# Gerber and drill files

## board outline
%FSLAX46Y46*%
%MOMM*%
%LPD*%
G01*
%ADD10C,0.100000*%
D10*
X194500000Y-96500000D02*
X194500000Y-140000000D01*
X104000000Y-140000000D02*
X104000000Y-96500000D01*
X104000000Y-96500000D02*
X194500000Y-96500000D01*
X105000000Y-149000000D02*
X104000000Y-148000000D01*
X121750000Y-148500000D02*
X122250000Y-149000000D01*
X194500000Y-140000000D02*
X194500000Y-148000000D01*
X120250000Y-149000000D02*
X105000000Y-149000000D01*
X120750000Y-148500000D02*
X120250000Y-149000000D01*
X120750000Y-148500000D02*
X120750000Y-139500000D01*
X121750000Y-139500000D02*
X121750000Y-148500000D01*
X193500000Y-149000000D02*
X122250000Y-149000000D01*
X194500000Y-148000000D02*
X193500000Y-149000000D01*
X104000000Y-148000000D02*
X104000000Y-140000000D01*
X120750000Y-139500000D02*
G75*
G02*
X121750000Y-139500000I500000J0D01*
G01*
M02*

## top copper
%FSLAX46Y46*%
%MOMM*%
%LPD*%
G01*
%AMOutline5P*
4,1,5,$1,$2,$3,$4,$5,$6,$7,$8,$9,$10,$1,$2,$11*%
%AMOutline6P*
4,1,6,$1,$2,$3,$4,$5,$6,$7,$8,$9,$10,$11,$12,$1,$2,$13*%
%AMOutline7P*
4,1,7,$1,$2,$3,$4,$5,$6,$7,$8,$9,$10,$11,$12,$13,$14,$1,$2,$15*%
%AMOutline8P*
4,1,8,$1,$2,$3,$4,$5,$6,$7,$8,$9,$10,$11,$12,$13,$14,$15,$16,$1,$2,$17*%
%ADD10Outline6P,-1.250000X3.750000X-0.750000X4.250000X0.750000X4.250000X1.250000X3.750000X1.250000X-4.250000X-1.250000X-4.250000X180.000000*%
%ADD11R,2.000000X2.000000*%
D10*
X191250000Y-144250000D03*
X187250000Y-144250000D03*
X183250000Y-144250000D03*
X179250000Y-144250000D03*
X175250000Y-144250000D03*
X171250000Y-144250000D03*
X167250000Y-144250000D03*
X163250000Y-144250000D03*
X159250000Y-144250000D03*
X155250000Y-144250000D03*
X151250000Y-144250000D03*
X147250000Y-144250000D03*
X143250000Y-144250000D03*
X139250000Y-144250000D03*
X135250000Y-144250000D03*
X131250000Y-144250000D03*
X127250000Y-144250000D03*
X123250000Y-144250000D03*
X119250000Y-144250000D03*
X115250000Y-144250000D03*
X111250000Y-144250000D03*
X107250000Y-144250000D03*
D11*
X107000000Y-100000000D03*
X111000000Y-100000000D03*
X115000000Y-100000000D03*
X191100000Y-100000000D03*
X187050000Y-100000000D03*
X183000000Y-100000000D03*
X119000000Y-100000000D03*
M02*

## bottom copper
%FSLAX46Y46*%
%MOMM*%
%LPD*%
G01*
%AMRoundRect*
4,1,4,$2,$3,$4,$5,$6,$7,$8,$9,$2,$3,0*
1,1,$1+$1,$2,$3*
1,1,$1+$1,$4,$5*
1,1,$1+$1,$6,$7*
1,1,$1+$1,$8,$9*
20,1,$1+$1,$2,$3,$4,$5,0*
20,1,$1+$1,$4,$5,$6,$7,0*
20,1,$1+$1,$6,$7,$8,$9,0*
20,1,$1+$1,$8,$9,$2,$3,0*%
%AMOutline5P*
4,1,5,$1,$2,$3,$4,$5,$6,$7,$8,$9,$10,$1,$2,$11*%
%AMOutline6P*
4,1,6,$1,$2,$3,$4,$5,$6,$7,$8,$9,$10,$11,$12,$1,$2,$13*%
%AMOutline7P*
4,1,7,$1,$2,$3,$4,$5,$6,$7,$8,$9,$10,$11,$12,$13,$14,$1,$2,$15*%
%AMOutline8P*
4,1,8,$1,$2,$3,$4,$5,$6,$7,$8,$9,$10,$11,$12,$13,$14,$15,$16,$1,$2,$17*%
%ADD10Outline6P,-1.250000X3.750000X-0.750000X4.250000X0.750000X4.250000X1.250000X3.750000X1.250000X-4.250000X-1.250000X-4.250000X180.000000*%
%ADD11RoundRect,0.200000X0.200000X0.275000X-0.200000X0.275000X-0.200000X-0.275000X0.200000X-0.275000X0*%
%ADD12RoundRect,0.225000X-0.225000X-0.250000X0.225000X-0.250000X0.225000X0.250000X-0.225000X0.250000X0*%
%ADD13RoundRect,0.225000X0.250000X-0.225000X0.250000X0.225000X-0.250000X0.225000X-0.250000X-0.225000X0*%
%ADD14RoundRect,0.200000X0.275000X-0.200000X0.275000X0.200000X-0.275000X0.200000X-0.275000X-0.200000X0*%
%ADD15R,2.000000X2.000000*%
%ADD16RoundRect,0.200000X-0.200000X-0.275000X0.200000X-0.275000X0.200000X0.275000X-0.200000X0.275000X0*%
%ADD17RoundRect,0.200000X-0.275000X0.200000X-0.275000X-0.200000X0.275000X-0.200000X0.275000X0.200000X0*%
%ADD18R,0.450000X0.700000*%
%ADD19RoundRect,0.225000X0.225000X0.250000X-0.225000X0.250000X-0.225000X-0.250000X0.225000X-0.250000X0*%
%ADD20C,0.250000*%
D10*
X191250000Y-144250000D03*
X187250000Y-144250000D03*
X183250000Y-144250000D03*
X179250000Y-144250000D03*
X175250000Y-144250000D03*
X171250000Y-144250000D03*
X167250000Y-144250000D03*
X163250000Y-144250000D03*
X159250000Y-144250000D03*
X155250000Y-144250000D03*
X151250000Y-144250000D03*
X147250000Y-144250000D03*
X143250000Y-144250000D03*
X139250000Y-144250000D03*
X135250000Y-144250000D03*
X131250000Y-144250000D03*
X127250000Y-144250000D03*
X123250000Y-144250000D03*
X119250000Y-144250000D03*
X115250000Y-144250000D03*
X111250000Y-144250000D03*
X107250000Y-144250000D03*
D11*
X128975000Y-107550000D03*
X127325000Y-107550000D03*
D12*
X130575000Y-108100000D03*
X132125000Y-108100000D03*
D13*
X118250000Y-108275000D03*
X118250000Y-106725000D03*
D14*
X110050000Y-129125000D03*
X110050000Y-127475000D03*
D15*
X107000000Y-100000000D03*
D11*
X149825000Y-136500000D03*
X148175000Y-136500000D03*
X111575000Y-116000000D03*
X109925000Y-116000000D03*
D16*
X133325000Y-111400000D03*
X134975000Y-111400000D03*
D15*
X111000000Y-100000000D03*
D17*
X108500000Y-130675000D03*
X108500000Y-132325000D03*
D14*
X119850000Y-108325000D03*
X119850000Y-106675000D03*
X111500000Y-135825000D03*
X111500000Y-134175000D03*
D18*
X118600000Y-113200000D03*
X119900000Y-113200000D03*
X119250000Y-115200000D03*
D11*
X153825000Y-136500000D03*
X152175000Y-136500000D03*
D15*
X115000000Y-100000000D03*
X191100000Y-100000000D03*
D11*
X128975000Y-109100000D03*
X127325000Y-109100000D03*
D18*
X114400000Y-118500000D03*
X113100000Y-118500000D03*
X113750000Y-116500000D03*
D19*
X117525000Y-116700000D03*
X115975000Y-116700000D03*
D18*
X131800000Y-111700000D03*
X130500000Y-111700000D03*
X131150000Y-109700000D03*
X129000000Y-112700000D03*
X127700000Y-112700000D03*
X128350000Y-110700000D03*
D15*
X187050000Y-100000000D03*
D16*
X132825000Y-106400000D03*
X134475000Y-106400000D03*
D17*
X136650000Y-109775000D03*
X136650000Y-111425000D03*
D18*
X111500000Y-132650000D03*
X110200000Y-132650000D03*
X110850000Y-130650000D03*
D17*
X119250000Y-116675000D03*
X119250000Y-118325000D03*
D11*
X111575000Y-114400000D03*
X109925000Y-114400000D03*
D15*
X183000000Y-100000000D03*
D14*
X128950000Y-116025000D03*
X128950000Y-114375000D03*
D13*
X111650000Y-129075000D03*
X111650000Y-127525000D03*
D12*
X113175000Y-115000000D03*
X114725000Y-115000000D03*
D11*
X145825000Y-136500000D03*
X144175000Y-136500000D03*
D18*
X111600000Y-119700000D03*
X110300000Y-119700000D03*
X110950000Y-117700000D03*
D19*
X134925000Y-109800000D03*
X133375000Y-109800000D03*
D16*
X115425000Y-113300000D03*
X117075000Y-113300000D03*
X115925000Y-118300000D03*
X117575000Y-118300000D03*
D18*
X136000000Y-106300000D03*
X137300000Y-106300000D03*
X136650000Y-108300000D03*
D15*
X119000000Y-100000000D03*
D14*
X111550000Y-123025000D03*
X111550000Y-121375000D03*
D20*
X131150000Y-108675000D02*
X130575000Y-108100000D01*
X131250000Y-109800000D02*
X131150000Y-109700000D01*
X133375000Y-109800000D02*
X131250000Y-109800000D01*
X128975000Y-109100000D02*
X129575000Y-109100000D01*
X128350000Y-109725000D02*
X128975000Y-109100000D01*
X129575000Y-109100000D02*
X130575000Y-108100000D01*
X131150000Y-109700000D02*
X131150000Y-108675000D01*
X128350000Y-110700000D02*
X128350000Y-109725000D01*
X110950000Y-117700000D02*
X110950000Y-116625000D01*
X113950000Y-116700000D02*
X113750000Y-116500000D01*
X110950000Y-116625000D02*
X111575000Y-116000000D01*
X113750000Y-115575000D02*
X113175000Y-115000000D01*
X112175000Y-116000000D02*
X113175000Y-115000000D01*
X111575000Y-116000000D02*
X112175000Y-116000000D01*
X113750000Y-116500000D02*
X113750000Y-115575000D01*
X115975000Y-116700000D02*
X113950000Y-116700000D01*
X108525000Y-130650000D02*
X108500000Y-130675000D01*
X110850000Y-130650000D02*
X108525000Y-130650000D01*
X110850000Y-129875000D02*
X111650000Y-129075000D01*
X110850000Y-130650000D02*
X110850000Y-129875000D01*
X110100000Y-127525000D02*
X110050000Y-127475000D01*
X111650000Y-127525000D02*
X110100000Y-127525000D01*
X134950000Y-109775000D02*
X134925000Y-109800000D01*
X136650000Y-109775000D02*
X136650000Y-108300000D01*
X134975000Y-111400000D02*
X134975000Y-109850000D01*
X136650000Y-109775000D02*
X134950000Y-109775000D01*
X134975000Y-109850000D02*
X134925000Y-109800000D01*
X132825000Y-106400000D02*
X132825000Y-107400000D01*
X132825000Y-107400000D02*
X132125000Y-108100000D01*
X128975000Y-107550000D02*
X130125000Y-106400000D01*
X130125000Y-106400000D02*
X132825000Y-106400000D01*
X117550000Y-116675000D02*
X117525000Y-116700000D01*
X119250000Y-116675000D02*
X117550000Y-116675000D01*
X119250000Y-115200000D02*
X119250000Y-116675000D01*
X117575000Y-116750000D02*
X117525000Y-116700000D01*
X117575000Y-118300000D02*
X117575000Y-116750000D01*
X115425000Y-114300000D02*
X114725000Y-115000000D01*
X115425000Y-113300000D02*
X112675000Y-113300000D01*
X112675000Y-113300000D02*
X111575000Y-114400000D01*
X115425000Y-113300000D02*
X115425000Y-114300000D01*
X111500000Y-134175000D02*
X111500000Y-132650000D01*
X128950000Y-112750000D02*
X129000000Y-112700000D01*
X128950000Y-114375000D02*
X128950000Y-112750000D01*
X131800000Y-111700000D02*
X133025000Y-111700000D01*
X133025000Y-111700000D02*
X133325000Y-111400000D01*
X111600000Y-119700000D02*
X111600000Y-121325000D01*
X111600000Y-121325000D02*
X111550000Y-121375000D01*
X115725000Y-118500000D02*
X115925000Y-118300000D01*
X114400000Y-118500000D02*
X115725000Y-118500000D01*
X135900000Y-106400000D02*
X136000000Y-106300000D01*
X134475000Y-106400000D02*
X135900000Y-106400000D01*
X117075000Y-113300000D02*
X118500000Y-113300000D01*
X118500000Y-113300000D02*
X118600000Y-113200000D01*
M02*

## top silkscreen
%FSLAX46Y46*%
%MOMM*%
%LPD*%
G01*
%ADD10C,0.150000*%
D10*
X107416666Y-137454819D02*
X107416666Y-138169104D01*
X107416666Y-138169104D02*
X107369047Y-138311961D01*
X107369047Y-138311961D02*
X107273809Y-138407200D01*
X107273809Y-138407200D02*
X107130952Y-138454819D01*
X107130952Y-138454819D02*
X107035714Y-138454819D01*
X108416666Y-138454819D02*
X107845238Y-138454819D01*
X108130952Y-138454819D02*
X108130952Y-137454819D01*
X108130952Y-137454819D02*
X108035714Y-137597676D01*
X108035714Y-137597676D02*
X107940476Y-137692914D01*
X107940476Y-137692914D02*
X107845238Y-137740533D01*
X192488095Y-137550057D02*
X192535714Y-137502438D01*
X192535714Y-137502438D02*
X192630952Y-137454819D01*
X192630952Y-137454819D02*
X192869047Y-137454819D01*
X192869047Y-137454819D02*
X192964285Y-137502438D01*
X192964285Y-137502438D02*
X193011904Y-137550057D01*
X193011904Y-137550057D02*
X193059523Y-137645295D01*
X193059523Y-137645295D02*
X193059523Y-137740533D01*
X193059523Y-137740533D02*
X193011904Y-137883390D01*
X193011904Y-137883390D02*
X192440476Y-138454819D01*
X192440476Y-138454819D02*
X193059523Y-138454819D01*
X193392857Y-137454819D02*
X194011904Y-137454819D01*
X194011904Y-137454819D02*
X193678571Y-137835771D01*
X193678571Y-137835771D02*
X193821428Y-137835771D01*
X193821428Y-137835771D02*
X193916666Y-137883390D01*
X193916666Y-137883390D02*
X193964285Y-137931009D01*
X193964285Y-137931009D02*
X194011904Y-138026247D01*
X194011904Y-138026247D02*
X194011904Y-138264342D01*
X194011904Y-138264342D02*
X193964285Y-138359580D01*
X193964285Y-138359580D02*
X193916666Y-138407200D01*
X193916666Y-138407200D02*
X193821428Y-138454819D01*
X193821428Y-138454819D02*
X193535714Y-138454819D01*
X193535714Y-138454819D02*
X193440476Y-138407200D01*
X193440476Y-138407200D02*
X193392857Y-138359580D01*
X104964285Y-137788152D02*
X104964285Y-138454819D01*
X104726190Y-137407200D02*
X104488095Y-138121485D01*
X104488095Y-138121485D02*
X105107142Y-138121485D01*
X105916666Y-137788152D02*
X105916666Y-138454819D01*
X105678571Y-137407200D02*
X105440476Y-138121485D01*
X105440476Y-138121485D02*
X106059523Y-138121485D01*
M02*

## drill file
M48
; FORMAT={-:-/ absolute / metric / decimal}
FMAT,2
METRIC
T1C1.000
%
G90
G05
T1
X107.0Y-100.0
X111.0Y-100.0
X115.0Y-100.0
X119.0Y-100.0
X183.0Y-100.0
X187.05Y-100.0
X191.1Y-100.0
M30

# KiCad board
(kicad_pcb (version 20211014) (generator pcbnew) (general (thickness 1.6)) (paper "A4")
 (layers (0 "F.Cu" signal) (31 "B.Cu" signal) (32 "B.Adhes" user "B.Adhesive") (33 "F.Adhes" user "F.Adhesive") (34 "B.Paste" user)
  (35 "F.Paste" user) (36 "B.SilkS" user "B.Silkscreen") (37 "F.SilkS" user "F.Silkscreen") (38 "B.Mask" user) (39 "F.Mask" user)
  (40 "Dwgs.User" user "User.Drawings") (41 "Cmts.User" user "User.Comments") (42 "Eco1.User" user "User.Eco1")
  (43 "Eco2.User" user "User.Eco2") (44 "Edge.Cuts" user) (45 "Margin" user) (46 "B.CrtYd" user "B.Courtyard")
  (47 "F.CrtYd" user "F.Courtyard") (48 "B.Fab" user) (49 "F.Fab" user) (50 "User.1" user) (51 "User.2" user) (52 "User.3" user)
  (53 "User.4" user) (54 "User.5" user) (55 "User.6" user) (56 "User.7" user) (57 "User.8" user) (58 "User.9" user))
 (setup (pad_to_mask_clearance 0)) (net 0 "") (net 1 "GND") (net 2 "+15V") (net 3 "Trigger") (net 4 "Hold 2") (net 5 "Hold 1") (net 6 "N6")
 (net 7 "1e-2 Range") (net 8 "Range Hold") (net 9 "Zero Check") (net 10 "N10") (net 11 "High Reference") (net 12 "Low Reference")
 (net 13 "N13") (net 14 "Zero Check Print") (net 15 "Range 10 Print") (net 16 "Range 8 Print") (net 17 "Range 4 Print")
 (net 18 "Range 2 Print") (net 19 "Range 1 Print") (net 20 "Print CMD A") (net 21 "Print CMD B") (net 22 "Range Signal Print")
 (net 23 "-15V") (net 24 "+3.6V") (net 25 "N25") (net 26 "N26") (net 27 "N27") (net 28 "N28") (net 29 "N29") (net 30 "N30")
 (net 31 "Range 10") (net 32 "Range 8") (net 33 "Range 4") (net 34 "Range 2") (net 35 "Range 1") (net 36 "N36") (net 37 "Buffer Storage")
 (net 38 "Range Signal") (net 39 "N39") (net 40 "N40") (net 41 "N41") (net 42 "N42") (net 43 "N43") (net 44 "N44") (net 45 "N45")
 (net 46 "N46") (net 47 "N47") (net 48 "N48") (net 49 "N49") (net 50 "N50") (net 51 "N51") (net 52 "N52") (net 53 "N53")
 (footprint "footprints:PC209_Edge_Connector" (layer "F.Cu") (at 104 140)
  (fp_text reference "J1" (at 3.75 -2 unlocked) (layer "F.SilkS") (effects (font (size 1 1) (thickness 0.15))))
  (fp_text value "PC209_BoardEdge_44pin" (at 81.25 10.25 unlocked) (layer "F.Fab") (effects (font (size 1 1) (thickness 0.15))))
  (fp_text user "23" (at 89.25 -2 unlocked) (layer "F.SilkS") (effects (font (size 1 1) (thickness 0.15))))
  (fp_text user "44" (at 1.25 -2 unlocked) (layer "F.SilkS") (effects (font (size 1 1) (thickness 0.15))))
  (fp_line (start 1 9) (end 0 8) (layer "Edge.Cuts") (width 0.1))
  (fp_line (start 17.75 8.5) (end 18.25 9) (layer "Edge.Cuts") (width 0.1))
  (fp_line (start 90.5 0) (end 90.5 8) (layer "Edge.Cuts") (width 0.1))
  (fp_line (start 16.25 9) (end 1 9) (layer "Edge.Cuts") (width 0.1))
  (fp_line (start 16.75 8.5) (end 16.25 9) (layer "Edge.Cuts") (width 0.1))
  (fp_line (start 16.75 8.5) (end 16.75 -0.5) (layer "Edge.Cuts") (width 0.1))
  (fp_line (start 17.75 -0.5) (end 17.75 8.5) (layer "Edge.Cuts") (width 0.1))
  (fp_line (start 89.5 9) (end 18.25 9) (layer "Edge.Cuts") (width 0.1))
  (fp_line (start 90.5 8) (end 89.5 9) (layer "Edge.Cuts") (width 0.1))
  (fp_line (start 0 8) (end 0 0) (layer "Edge.Cuts") (width 0.1))
  (fp_arc (start 16.75 -0.5) (mid 17.25 -1) (end 17.75 -0.5) (layer "Edge.Cuts") (width 0.1))
  (pad "1" connect roundrect (at 87.25 4.25 180) (size 2.5 8.5) (layers "B.Cu" "B.Mask") (roundrect_rratio 0) (chamfer_ratio 0.2)
   (chamfer top_left top_right) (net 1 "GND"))
  (pad "2" connect roundrect (at 83.25 4.25 180) (size 2.5 8.5) (layers "B.Cu" "B.Mask") (roundrect_rratio 0) (chamfer_ratio 0.2)
   (chamfer top_left top_right) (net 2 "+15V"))
  (pad "3" connect roundrect (at 79.25 4.25 180) (size 2.5 8.5) (layers "B.Cu" "B.Mask") (roundrect_rratio 0) (chamfer_ratio 0.2)
   (chamfer top_left top_right) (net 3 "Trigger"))
  (pad "4" connect roundrect (at 75.25 4.25 180) (size 2.5 8.5) (layers "B.Cu" "B.Mask") (roundrect_rratio 0) (chamfer_ratio 0.2)
   (chamfer top_left top_right) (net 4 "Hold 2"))
  (pad "5" connect roundrect (at 71.25 4.25 180) (size 2.5 8.5) (layers "B.Cu" "B.Mask") (roundrect_rratio 0) (chamfer_ratio 0.2)
   (chamfer top_left top_right) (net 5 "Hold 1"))
  (pad "6" connect roundrect (at 67.25 4.25 180) (size 2.5 8.5) (layers "B.Cu" "B.Mask") (roundrect_rratio 0) (chamfer_ratio 0.2)
   (chamfer top_left top_right) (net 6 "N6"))
  (pad "7" connect roundrect (at 63.25 4.25 180) (size 2.5 8.5) (layers "B.Cu" "B.Mask") (roundrect_rratio 0) (chamfer_ratio 0.2)
   (chamfer top_left top_right) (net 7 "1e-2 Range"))
  (pad "8" connect roundrect (at 59.25 4.25 180) (size 2.5 8.5) (layers "B.Cu" "B.Mask") (roundrect_rratio 0) (chamfer_ratio 0.2)
   (chamfer top_left top_right) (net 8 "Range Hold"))
  (pad "9" connect roundrect (at 55.25 4.25 180) (size 2.5 8.5) (layers "B.Cu" "B.Mask") (roundrect_rratio 0) (chamfer_ratio 0.2)
   (chamfer top_left top_right) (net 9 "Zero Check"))
  (pad "10" connect roundrect (at 51.25 4.25 180) (size 2.5 8.5) (layers "B.Cu" "B.Mask") (roundrect_rratio 0) (chamfer_ratio 0.2)
   (chamfer top_left top_right) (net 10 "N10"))
  (pad "11" connect roundrect (at 47.25 4.25 180) (size 2.5 8.5) (layers "B.Cu" "B.Mask") (roundrect_rratio 0) (chamfer_ratio 0.2)
   (chamfer top_left top_right) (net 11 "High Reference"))
  (pad "12" connect roundrect (at 43.25 4.25 180) (size 2.5 8.5) (layers "B.Cu" "B.Mask") (roundrect_rratio 0) (chamfer_ratio 0.2)
   (chamfer top_left top_right) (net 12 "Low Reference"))
  (pad "13" connect roundrect (at 39.25 4.25 180) (size 2.5 8.5) (layers "B.Cu" "B.Mask") (roundrect_rratio 0) (chamfer_ratio 0.2)
   (chamfer top_left top_right) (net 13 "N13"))
  (pad "14" connect roundrect (at 35.25 4.25 180) (size 2.5 8.5) (layers "B.Cu" "B.Mask") (roundrect_rratio 0) (chamfer_ratio 0.2)
   (chamfer top_left top_right) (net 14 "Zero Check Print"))
  (pad "15" connect roundrect (at 31.25 4.25 180) (size 2.5 8.5) (layers "B.Cu" "B.Mask") (roundrect_rratio 0) (chamfer_ratio 0.2)
   (chamfer top_left top_right) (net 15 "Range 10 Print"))
  (pad "16" connect roundrect (at 27.25 4.25 180) (size 2.5 8.5) (layers "B.Cu" "B.Mask") (roundrect_rratio 0) (chamfer_ratio 0.2)
   (chamfer top_left top_right) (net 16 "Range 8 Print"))
  (pad "17" connect roundrect (at 23.25 4.25 180) (size 2.5 8.5) (layers "B.Cu" "B.Mask") (roundrect_rratio 0) (chamfer_ratio 0.2)
   (chamfer top_left top_right) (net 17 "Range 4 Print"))
  (pad "18" connect roundrect (at 19.25 4.25 180) (size 2.5 8.5) (layers "B.Cu" "B.Mask") (roundrect_rratio 0) (chamfer_ratio 0.2)
   (chamfer top_left top_right) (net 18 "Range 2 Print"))
  (pad "19" connect roundrect (at 15.25 4.25 180) (size 2.5 8.5) (layers "B.Cu" "B.Mask") (roundrect_rratio 0) (chamfer_ratio 0.2)
   (chamfer top_left top_right) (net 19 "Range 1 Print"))
  (pad "20" connect roundrect (at 11.25 4.25 180) (size 2.5 8.5) (layers "B.Cu" "B.Mask") (roundrect_rratio 0) (chamfer_ratio 0.2)
   (chamfer top_left top_right) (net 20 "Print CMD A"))
  (pad "21" connect roundrect (at 7.25 4.25 180) (size 2.5 8.5) (layers "B.Cu" "B.Mask") (roundrect_rratio 0) (chamfer_ratio 0.2)
   (chamfer top_left top_right) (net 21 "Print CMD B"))
  (pad "22" connect roundrect (at 3.25 4.25 180) (size 2.5 8.5) (layers "B.Cu" "B.Mask") (roundrect_rratio 0) (chamfer_ratio 0.2)
   (chamfer top_left top_right) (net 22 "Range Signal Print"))
  (pad "23" connect roundrect (at 87.25 4.25 180) (size 2.5 8.5) (layers "F.Cu" "F.Mask") (roundrect_rratio 0) (chamfer_ratio 0.2)
   (chamfer top_left top_right) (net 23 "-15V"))
  (pad "24" connect roundrect (at 83.25 4.25 180) (size 2.5 8.5) (layers "F.Cu" "F.Mask") (roundrect_rratio 0) (chamfer_ratio 0.2)
   (chamfer top_left top_right) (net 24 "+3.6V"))
  (pad "25" connect roundrect (at 79.25 4.25 180) (size 2.5 8.5) (layers "F.Cu" "F.Mask") (roundrect_rratio 0) (chamfer_ratio 0.2)
   (chamfer top_left top_right) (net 3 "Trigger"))
  (pad "26" connect roundrect (at 75.25 4.25 180) (size 2.5 8.5) (layers "F.Cu" "F.Mask") (roundrect_rratio 0) (chamfer_ratio 0.2)
   (chamfer top_left top_right) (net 4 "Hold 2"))
  (pad "27" connect roundrect (at 71.25 4.25 180) (size 2.5 8.5) (layers "F.Cu" "F.Mask") (roundrect_rratio 0) (chamfer_ratio 0.2)
   (chamfer top_left top_right) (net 5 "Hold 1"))
  (pad "28" connect roundrect (at 67.25 4.25 180) (size 2.5 8.5) (layers "F.Cu" "F.Mask") (roundrect_rratio 0) (chamfer_ratio 0.2)
   (chamfer top_left top_right) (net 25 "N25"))
  (pad "29" connect roundrect (at 63.25 4.25 180) (size 2.5 8.5) (layers "F.Cu" "F.Mask") (roundrect_rratio 0) (chamfer_ratio 0.2)
   (chamfer top_left top_right) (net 7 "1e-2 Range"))
  (pad "30" connect roundrect (at 59.25 4.25 180) (size 2.5 8.5) (layers "F.Cu" "F.Mask") (roundrect_rratio 0) (chamfer_ratio 0.2)
   (chamfer top_left top_right) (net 8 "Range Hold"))
  (pad "31" connect roundrect (at 55.25 4.25 180) (size 2.5 8.5) (layers "F.Cu" "F.Mask") (roundrect_rratio 0) (chamfer_ratio 0.2)
   (chamfer top_left top_right) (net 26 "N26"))
  (pad "32" connect roundrect (at 51.25 4.25 180) (size 2.5 8.5) (layers "F.Cu" "F.Mask") (roundrect_rratio 0) (chamfer_ratio 0.2)
   (chamfer top_left top_right) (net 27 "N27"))
  (pad "33" connect roundrect (at 47.25 4.25 180) (size 2.5 8.5) (layers "F.Cu" "F.Mask") (roundrect_rratio 0) (chamfer_ratio 0.2)
   (chamfer top_left top_right) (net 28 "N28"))
  (pad "34" connect roundrect (at 43.25 4.25 180) (size 2.5 8.5) (layers "F.Cu" "F.Mask") (roundrect_rratio 0) (chamfer_ratio 0.2)
   (chamfer top_left top_right) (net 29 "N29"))
  (pad "35" connect roundrect (at 39.25 4.25 180) (size 2.5 8.5) (layers "F.Cu" "F.Mask") (roundrect_rratio 0) (chamfer_ratio 0.2)
   (chamfer top_left top_right) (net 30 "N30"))
  (pad "36" connect roundrect (at 35.25 4.25 180) (size 2.5 8.5) (layers "F.Cu" "F.Mask") (roundrect_rratio 0) (chamfer_ratio 0.2)
   (chamfer top_left top_right) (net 9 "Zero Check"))
  (pad "37" connect roundrect (at 31.25 4.25 180) (size 2.5 8.5) (layers "F.Cu" "F.Mask") (roundrect_rratio 0) (chamfer_ratio 0.2)
   (chamfer top_left top_right) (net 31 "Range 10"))
  (pad "38" connect roundrect (at 27.25 4.25 180) (size 2.5 8.5) (layers "F.Cu" "F.Mask") (roundrect_rratio 0) (chamfer_ratio 0.2)
   (chamfer top_left top_right) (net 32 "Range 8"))
  (pad "39" connect roundrect (at 23.25 4.25 180) (size 2.5 8.5) (layers "F.Cu" "F.Mask") (roundrect_rratio 0) (chamfer_ratio 0.2)
   (chamfer top_left top_right) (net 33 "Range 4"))
  (pad "40" connect roundrect (at 19.25 4.25 180) (size 2.5 8.5) (layers "F.Cu" "F.Mask") (roundrect_rratio 0) (chamfer_ratio 0.2)
   (chamfer top_left top_right) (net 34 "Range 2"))
  (pad "41" connect roundrect (at 15.25 4.25 180) (size 2.5 8.5) (layers "F.Cu" "F.Mask") (roundrect_rratio 0) (chamfer_ratio 0.2)
   (chamfer top_left top_right) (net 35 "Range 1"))
  (pad "42" connect roundrect (at 11.25 4.25 180) (size 2.5 8.5) (layers "F.Cu" "F.Mask") (roundrect_rratio 0) (chamfer_ratio 0.2)
   (chamfer top_left top_right) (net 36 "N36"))
  (pad "43" connect roundrect (at 7.25 4.25 180) (size 2.5 8.5) (layers "F.Cu" "F.Mask") (roundrect_rratio 0) (chamfer_ratio 0.2)
   (chamfer top_left top_right) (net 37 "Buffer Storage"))
  (pad "44" connect roundrect (at 3.25 4.25 180) (size 2.5 8.5) (layers "F.Cu" "F.Mask") (roundrect_rratio 0) (chamfer_ratio 0.2)
   (chamfer top_left top_right) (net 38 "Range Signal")))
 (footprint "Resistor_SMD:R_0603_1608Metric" (layer "B.Cu") (at 128.15 107.55 180)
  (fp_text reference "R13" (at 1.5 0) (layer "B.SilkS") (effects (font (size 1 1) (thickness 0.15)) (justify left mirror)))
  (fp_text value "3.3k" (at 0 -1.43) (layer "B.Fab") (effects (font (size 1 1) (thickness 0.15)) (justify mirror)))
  (pad "1" smd roundrect (at -0.825 0 180) (size 0.8 0.95) (layers "B.Cu" "B.Paste" "B.Mask") (roundrect_rratio 0.25) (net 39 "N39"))
  (pad "2" smd roundrect (at 0.825 0 180) (size 0.8 0.95) (layers "B.Cu" "B.Paste" "B.Mask") (roundrect_rratio 0.25) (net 24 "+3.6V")))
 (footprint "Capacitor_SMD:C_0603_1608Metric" (layer "B.Cu") (at 131.35 108.1)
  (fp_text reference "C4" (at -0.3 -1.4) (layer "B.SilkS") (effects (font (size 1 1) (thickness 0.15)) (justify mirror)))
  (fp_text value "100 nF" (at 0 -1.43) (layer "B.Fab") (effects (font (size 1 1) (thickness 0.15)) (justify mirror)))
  (pad "1" smd roundrect (at -0.775 0) (size 0.9 0.95) (layers "B.Cu" "B.Paste" "B.Mask") (roundrect_rratio 0.25) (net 20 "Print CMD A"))
  (pad "2" smd roundrect (at 0.775 0) (size 0.9 0.95) (layers "B.Cu" "B.Paste" "B.Mask") (roundrect_rratio 0.25) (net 39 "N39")))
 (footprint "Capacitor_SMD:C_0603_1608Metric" (layer "B.Cu") (at 118.25 107.5 90)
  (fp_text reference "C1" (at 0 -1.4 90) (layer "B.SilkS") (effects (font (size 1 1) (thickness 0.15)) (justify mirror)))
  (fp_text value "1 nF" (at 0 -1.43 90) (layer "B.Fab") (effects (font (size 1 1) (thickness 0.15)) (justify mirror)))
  (pad "1" smd roundrect (at -0.775 0 90) (size 0.9 0.95) (layers "B.Cu" "B.Paste" "B.Mask") (roundrect_rratio 0.25) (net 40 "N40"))
  (pad "2" smd roundrect (at 0.775 0 90) (size 0.9 0.95) (layers "B.Cu" "B.Paste" "B.Mask") (roundrect_rratio 0.25) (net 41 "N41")))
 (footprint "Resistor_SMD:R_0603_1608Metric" (layer "B.Cu") (at 110.05 128.3 90)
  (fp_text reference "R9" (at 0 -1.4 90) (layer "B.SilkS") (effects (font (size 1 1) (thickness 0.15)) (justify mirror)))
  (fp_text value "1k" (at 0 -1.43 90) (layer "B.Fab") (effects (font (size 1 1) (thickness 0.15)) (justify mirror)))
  (pad "1" smd roundrect (at -0.825 0 90) (size 0.8 0.95) (layers "B.Cu" "B.Paste" "B.Mask") (roundrect_rratio 0.25) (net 1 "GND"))
  (pad "2" smd roundrect (at 0.825 0 90) (size 0.8 0.95) (layers "B.Cu" "B.Paste" "B.Mask") (roundrect_rratio 0.25) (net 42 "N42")))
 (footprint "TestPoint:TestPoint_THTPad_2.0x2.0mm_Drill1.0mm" (layer "B.Cu") (at 107 100 180)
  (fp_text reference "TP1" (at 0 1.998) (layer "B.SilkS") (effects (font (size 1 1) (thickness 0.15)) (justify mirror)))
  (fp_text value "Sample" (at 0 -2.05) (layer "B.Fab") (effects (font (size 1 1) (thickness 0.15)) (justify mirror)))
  (pad "1" thru_hole rect (at 0 0 180) (size 2 2) (drill 1) (layers *.Cu *.Mask) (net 37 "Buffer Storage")))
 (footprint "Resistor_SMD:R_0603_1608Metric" (layer "B.Cu") (at 149 136.5 180)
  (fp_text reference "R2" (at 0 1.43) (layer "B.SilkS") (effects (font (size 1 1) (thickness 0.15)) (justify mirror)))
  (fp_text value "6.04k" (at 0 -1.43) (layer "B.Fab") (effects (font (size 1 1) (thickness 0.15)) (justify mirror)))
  (pad "1" smd roundrect (at -0.825 0 180) (size 0.8 0.95) (layers "B.Cu" "B.Paste" "B.Mask") (roundrect_rratio 0.25)
   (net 11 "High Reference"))
  (pad "2" smd roundrect (at 0.825 0 180) (size 0.8 0.95) (layers "B.Cu" "B.Paste" "B.Mask") (roundrect_rratio 0.25)
   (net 12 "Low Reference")))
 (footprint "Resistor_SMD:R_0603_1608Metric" (layer "B.Cu") (at 110.75 116 180)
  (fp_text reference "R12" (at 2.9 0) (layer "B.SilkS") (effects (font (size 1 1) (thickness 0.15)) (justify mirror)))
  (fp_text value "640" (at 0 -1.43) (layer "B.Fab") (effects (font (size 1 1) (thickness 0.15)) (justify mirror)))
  (pad "1" smd roundrect (at -0.825 0 180) (size 0.8 0.95) (layers "B.Cu" "B.Paste" "B.Mask") (roundrect_rratio 0.25) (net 40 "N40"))
  (pad "2" smd roundrect (at 0.825 0 180) (size 0.8 0.95) (layers "B.Cu" "B.Paste" "B.Mask") (roundrect_rratio 0.25) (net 24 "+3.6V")))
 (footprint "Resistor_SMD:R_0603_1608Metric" (layer "B.Cu") (at 134.15 111.4)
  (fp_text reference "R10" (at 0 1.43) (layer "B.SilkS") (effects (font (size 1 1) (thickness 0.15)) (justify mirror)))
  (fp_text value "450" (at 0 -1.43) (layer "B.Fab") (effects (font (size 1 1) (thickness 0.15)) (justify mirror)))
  (pad "1" smd roundrect (at -0.825 0) (size 0.8 0.95) (layers "B.Cu" "B.Paste" "B.Mask") (roundrect_rratio 0.25) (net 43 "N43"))
  (pad "2" smd roundrect (at 0.825 0) (size 0.8 0.95) (layers "B.Cu" "B.Paste" "B.Mask") (roundrect_rratio 0.25) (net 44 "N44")))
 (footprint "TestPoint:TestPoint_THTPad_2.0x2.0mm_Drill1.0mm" (layer "B.Cu") (at 111 100 180)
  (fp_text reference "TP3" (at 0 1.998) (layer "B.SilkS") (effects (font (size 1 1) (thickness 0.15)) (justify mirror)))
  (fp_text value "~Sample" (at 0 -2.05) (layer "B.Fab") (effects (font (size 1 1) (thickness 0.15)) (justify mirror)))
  (pad "1" thru_hole rect (at 0 0 180) (size 2 2) (drill 1) (layers *.Cu *.Mask) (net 42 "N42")))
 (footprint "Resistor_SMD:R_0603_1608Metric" (layer "B.Cu") (at 108.5 131.5 -90)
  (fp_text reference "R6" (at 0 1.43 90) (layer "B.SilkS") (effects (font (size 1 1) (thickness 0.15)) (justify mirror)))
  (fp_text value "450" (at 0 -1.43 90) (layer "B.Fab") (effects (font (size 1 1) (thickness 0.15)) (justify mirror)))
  (pad "1" smd roundrect (at -0.825 0 270) (size 0.8 0.95) (layers "B.Cu" "B.Paste" "B.Mask") (roundrect_rratio 0.25) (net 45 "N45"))
  (pad "2" smd roundrect (at 0.825 0 270) (size 0.8 0.95) (layers "B.Cu" "B.Paste" "B.Mask") (roundrect_rratio 0.25) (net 24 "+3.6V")))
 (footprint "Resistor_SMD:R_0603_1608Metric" (layer "B.Cu") (at 119.85 107.5 90)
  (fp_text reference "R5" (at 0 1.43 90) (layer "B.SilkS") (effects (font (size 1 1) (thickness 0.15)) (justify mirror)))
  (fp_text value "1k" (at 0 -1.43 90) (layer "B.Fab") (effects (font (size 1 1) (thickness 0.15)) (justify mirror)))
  (pad "1" smd roundrect (at -0.825 0 90) (size 0.8 0.95) (layers "B.Cu" "B.Paste" "B.Mask") (roundrect_rratio 0.25) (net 1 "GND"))
  (pad "2" smd roundrect (at 0.825 0 90) (size 0.8 0.95) (layers "B.Cu" "B.Paste" "B.Mask") (roundrect_rratio 0.25) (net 41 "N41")))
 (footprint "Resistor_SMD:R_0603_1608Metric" (layer "B.Cu") (at 111.5 135 90)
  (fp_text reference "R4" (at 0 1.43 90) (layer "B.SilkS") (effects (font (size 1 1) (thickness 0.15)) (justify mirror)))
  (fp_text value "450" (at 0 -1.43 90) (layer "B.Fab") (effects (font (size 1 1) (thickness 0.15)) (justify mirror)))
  (pad "1" smd roundrect (at -0.825 0 90) (size 0.8 0.95) (layers "B.Cu" "B.Paste" "B.Mask") (roundrect_rratio 0.25)
   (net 37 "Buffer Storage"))
  (pad "2" smd roundrect (at 0.825 0 90) (size 0.8 0.95) (layers "B.Cu" "B.Paste" "B.Mask") (roundrect_rratio 0.25) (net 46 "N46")))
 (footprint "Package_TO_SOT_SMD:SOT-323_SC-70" (layer "B.Cu") (at 119.25 114.2 -90)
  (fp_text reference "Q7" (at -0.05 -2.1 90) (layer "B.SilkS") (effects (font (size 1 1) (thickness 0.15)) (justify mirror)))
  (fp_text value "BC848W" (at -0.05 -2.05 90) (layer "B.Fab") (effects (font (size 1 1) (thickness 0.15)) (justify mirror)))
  (pad "1" smd rect (at -1 0.65) (size 0.45 0.7) (layers "B.Cu" "B.Paste" "B.Mask") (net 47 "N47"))
  (pad "2" smd rect (at -1 -0.65) (size 0.45 0.7) (layers "B.Cu" "B.Paste" "B.Mask") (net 1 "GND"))
  (pad "3" smd rect (at 1 0) (size 0.45 0.7) (layers "B.Cu" "B.Paste" "B.Mask") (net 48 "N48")))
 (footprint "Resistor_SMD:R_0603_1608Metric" (layer "B.Cu") (at 153 136.5 180)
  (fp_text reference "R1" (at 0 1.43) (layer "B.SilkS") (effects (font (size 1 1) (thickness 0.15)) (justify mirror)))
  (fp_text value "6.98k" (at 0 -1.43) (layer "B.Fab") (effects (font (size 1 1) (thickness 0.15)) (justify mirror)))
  (pad "1" smd roundrect (at -0.825 0 180) (size 0.8 0.95) (layers "B.Cu" "B.Paste" "B.Mask") (roundrect_rratio 0.25) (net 2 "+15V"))
  (pad "2" smd roundrect (at 0.825 0 180) (size 0.8 0.95) (layers "B.Cu" "B.Paste" "B.Mask") (roundrect_rratio 0.25)
   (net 11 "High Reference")))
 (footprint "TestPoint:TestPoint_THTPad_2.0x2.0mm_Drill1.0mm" (layer "B.Cu") (at 115 100 180)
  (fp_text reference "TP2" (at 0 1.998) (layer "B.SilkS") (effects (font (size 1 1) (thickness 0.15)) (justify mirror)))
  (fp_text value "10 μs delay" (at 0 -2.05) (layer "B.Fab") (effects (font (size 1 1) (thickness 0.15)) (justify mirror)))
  (pad "1" thru_hole rect (at 0 0 180) (size 2 2) (drill 1) (layers *.Cu *.Mask) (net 40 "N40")))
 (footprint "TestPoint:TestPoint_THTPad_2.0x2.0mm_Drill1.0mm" (layer "B.Cu") (at 191.1 100 180)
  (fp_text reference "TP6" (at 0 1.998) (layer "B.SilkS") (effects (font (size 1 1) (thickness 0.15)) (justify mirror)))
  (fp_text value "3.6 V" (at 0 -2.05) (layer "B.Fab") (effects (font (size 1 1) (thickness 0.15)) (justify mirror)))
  (pad "1" thru_hole rect (at 0 0 180) (size 2 2) (drill 1) (layers *.Cu *.Mask) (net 24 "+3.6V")))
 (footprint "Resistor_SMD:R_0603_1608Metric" (layer "B.Cu") (at 128.15 109.1 180)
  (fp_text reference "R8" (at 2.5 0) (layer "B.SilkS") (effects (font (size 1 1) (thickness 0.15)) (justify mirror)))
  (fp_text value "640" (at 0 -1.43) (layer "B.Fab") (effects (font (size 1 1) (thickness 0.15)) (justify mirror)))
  (pad "1" smd roundrect (at -0.825 0 180) (size 0.8 0.95) (layers "B.Cu" "B.Paste" "B.Mask") (roundrect_rratio 0.25) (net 20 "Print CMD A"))
  (pad "2" smd roundrect (at 0.825 0 180) (size 0.8 0.95) (layers "B.Cu" "B.Paste" "B.Mask") (roundrect_rratio 0.25) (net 24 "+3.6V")))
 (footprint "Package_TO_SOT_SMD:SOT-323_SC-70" (layer "B.Cu") (at 113.75 117.5 90)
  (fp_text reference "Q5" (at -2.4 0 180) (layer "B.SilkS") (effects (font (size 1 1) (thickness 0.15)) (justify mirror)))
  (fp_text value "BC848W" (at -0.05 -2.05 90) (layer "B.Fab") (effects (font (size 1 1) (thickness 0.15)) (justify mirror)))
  (pad "1" smd rect (at -1 0.65 180) (size 0.45 0.7) (layers "B.Cu" "B.Paste" "B.Mask") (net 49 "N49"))
  (pad "2" smd rect (at -1 -0.65 180) (size 0.45 0.7) (layers "B.Cu" "B.Paste" "B.Mask") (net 1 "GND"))
  (pad "3" smd rect (at 1 0 180) (size 0.45 0.7) (layers "B.Cu" "B.Paste" "B.Mask") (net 40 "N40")))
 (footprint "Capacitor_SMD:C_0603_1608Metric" (layer "B.Cu") (at 116.75 116.7 180)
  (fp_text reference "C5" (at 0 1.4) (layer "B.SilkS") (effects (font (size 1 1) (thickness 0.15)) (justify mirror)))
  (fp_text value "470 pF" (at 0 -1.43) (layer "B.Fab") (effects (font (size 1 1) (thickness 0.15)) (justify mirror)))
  (pad "1" smd roundrect (at -0.775 0 180) (size 0.9 0.95) (layers "B.Cu" "B.Paste" "B.Mask") (roundrect_rratio 0.25) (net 48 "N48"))
  (pad "2" smd roundrect (at 0.775 0 180) (size 0.9 0.95) (layers "B.Cu" "B.Paste" "B.Mask") (roundrect_rratio 0.25) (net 40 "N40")))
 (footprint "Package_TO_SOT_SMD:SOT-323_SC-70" (layer "B.Cu") (at 131.15 110.7 90)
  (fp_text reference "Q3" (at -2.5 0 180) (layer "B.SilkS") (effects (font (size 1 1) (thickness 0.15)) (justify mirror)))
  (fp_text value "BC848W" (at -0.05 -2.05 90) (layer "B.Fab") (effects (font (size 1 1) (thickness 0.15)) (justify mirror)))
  (pad "1" smd rect (at -1 0.65 180) (size 0.45 0.7) (layers "B.Cu" "B.Paste" "B.Mask") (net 43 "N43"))
  (pad "2" smd rect (at -1 -0.65 180) (size 0.45 0.7) (layers "B.Cu" "B.Paste" "B.Mask") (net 1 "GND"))
  (pad "3" smd rect (at 1 0 180) (size 0.45 0.7) (layers "B.Cu" "B.Paste" "B.Mask") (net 20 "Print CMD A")))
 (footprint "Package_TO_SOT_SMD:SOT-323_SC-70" (layer "B.Cu") (at 128.35 111.7 90)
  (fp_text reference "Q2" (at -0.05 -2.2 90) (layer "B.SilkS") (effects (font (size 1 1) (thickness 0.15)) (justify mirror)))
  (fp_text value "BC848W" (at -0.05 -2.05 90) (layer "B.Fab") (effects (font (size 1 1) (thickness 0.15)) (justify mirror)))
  (pad "1" smd rect (at -1 0.65 180) (size 0.45 0.7) (layers "B.Cu" "B.Paste" "B.Mask") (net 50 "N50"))
  (pad "2" smd rect (at -1 -0.65 180) (size 0.45 0.7) (layers "B.Cu" "B.Paste" "B.Mask") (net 1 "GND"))
  (pad "3" smd rect (at 1 0 180) (size 0.45 0.7) (layers "B.Cu" "B.Paste" "B.Mask") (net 20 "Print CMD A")))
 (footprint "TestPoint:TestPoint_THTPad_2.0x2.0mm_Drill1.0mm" (layer "B.Cu") (at 187.05 100 180)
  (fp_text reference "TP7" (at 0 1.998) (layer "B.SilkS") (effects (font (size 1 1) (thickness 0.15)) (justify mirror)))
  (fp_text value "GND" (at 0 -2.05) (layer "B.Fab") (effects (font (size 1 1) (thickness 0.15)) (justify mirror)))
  (pad "1" thru_hole rect (at 0 0 180) (size 2 2) (drill 1) (layers *.Cu *.Mask) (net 1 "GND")))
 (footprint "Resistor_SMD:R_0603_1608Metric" (layer "B.Cu") (at 133.65 106.4)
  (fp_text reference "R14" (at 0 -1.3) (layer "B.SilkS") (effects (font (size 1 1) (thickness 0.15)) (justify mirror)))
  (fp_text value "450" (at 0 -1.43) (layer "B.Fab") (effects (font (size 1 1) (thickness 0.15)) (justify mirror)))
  (pad "1" smd roundrect (at -0.825 0) (size 0.8 0.95) (layers "B.Cu" "B.Paste" "B.Mask") (roundrect_rratio 0.25) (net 39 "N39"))
  (pad "2" smd roundrect (at 0.825 0) (size 0.8 0.95) (layers "B.Cu" "B.Paste" "B.Mask") (roundrect_rratio 0.25) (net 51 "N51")))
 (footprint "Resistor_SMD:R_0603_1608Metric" (layer "B.Cu") (at 136.65 110.6 -90)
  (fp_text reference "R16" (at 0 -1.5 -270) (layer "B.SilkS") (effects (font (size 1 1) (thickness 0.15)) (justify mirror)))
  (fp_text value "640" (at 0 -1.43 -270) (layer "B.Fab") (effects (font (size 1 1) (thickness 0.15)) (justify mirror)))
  (pad "1" smd roundrect (at -0.825 0 270) (size 0.8 0.95) (layers "B.Cu" "B.Paste" "B.Mask") (roundrect_rratio 0.25) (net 44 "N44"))
  (pad "2" smd roundrect (at 0.825 0 270) (size 0.8 0.95) (layers "B.Cu" "B.Paste" "B.Mask") (roundrect_rratio 0.25) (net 24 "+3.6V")))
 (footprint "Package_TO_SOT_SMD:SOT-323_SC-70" (layer "B.Cu") (at 110.85 131.65 90)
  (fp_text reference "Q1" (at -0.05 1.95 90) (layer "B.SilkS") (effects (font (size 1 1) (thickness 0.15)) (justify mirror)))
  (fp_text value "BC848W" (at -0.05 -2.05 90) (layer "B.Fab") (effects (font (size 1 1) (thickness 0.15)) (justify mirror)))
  (pad "1" smd rect (at -1 0.65 180) (size 0.45 0.7) (layers "B.Cu" "B.Paste" "B.Mask") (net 46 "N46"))
  (pad "2" smd rect (at -1 -0.65 180) (size 0.45 0.7) (layers "B.Cu" "B.Paste" "B.Mask") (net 1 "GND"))
  (pad "3" smd rect (at 1 0 180) (size 0.45 0.7) (layers "B.Cu" "B.Paste" "B.Mask") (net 45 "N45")))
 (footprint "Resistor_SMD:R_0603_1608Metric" (layer "B.Cu") (at 119.25 117.5 -90)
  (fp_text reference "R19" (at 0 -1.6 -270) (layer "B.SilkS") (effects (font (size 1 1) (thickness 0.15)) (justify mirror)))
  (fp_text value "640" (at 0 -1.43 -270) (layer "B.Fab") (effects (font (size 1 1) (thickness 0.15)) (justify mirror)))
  (pad "1" smd roundrect (at -0.825 0 270) (size 0.8 0.95) (layers "B.Cu" "B.Paste" "B.Mask") (roundrect_rratio 0.25) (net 48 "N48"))
  (pad "2" smd roundrect (at 0.825 0 270) (size 0.8 0.95) (layers "B.Cu" "B.Paste" "B.Mask") (roundrect_rratio 0.25) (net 24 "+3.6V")))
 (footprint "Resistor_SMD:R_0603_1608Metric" (layer "B.Cu") (at 110.75 114.4 180)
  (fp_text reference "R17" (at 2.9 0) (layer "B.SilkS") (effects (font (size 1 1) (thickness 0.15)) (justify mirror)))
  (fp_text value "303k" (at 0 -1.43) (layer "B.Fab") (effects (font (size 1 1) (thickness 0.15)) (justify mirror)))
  (pad "1" smd roundrect (at -0.825 0 180) (size 0.8 0.95) (layers "B.Cu" "B.Paste" "B.Mask") (roundrect_rratio 0.25) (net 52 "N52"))
  (pad "2" smd roundrect (at 0.825 0 180) (size 0.8 0.95) (layers "B.Cu" "B.Paste" "B.Mask") (roundrect_rratio 0.25) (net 24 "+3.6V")))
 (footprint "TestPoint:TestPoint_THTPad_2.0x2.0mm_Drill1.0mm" (layer "B.Cu") (at 183 100 180)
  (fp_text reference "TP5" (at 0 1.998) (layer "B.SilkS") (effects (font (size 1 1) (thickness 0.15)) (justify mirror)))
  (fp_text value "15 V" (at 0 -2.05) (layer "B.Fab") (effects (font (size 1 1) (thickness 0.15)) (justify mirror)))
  (pad "1" thru_hole rect (at 0 0 180) (size 2 2) (drill 1) (layers *.Cu *.Mask) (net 2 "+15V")))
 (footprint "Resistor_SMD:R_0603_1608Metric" (layer "B.Cu") (at 128.95 115.2 90)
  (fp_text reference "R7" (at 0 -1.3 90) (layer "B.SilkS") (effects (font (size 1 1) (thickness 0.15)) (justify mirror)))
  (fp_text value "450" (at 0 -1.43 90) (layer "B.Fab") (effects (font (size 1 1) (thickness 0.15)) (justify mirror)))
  (pad "1" smd roundrect (at -0.825 0 90) (size 0.8 0.95) (layers "B.Cu" "B.Paste" "B.Mask") (roundrect_rratio 0.25) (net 41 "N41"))
  (pad "2" smd roundrect (at 0.825 0 90) (size 0.8 0.95) (layers "B.Cu" "B.Paste" "B.Mask") (roundrect_rratio 0.25) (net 50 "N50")))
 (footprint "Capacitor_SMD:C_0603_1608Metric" (layer "B.Cu") (at 111.65 128.3 90)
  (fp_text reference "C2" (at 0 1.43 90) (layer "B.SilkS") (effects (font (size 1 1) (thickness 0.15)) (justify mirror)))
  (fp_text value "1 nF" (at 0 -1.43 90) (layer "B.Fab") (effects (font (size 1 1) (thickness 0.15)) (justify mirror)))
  (pad "1" smd roundrect (at -0.775 0 90) (size 0.9 0.95) (layers "B.Cu" "B.Paste" "B.Mask") (roundrect_rratio 0.25) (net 45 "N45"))
  (pad "2" smd roundrect (at 0.775 0 90) (size 0.9 0.95) (layers "B.Cu" "B.Paste" "B.Mask") (roundrect_rratio 0.25) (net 42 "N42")))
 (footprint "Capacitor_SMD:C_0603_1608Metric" (layer "B.Cu") (at 113.95 115)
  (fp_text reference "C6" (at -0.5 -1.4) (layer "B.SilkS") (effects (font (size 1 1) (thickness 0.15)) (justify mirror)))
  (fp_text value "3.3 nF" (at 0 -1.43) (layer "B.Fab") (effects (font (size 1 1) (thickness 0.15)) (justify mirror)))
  (pad "1" smd roundrect (at -0.775 0) (size 0.9 0.95) (layers "B.Cu" "B.Paste" "B.Mask") (roundrect_rratio 0.25) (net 40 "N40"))
  (pad "2" smd roundrect (at 0.775 0) (size 0.9 0.95) (layers "B.Cu" "B.Paste" "B.Mask") (roundrect_rratio 0.25) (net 52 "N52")))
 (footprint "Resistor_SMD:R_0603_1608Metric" (layer "B.Cu") (at 145 136.5 180)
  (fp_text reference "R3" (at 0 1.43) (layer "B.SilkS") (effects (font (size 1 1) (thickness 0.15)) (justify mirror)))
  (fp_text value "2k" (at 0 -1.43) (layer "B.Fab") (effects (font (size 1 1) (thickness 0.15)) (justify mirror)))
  (pad "1" smd roundrect (at -0.825 0 180) (size 0.8 0.95) (layers "B.Cu" "B.Paste" "B.Mask") (roundrect_rratio 0.25)
   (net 12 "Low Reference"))
  (pad "2" smd roundrect (at 0.825 0 180) (size 0.8 0.95) (layers "B.Cu" "B.Paste" "B.Mask") (roundrect_rratio 0.25) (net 1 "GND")))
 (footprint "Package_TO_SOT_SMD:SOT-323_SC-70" (layer "B.Cu") (at 110.95 118.7 90)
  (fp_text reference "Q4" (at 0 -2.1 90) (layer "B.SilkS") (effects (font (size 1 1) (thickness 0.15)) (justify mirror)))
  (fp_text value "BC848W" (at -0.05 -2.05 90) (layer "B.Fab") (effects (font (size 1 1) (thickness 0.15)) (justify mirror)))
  (pad "1" smd rect (at -1 0.65 180) (size 0.45 0.7) (layers "B.Cu" "B.Paste" "B.Mask") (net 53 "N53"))
  (pad "2" smd rect (at -1 -0.65 180) (size 0.45 0.7) (layers "B.Cu" "B.Paste" "B.Mask") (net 1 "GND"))
  (pad "3" smd rect (at 1 0 180) (size 0.45 0.7) (layers "B.Cu" "B.Paste" "B.Mask") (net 40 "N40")))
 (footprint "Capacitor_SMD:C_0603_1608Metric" (layer "B.Cu") (at 134.15 109.8 180)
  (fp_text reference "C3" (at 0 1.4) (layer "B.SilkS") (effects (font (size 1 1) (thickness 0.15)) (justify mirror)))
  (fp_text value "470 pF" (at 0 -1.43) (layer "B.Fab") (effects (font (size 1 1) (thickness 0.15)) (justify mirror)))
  (pad "1" smd roundrect (at -0.775 0 180) (size 0.9 0.95) (layers "B.Cu" "B.Paste" "B.Mask") (roundrect_rratio 0.25) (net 44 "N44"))
  (pad "2" smd roundrect (at 0.775 0 180) (size 0.9 0.95) (layers "B.Cu" "B.Paste" "B.Mask") (roundrect_rratio 0.25) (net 20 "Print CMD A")))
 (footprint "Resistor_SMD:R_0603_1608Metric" (layer "B.Cu") (at 116.25 113.3)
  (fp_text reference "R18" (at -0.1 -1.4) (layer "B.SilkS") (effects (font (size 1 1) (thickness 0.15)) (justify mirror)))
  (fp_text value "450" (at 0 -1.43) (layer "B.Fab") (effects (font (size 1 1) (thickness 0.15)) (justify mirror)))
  (pad "1" smd roundrect (at -0.825 0) (size 0.8 0.95) (layers "B.Cu" "B.Paste" "B.Mask") (roundrect_rratio 0.25) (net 52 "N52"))
  (pad "2" smd roundrect (at 0.825 0) (size 0.8 0.95) (layers "B.Cu" "B.Paste" "B.Mask") (roundrect_rratio 0.25) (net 47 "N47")))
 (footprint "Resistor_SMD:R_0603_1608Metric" (layer "B.Cu") (at 116.75 118.3)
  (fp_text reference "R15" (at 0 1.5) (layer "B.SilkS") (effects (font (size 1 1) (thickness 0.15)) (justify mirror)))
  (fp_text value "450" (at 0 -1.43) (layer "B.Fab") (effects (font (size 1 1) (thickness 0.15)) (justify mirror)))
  (pad "1" smd roundrect (at -0.825 0) (size 0.8 0.95) (layers "B.Cu" "B.Paste" "B.Mask") (roundrect_rratio 0.25) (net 49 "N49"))
  (pad "2" smd roundrect (at 0.825 0) (size 0.8 0.95) (layers "B.Cu" "B.Paste" "B.Mask") (roundrect_rratio 0.25) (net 48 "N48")))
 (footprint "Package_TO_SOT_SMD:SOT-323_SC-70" (layer "B.Cu") (at 136.65 107.3 -90)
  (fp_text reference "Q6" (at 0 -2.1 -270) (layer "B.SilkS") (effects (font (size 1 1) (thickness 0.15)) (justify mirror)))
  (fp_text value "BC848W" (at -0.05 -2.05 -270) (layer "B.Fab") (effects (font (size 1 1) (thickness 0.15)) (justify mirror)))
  (pad "1" smd rect (at -1 0.65) (size 0.45 0.7) (layers "B.Cu" "B.Paste" "B.Mask") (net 51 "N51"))
  (pad "2" smd rect (at -1 -0.65) (size 0.45 0.7) (layers "B.Cu" "B.Paste" "B.Mask") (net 1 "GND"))
  (pad "3" smd rect (at 1 0) (size 0.45 0.7) (layers "B.Cu" "B.Paste" "B.Mask") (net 44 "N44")))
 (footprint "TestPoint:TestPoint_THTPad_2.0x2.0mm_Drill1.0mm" (layer "B.Cu") (at 119 100 180)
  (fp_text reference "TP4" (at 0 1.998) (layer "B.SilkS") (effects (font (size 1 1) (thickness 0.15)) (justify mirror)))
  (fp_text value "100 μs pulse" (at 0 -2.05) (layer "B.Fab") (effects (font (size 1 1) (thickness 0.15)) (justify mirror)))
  (pad "1" thru_hole rect (at 0 0 180) (size 2 2) (drill 1) (layers *.Cu *.Mask) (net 20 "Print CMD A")))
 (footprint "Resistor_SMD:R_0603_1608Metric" (layer "B.Cu") (at 111.55 122.2 90)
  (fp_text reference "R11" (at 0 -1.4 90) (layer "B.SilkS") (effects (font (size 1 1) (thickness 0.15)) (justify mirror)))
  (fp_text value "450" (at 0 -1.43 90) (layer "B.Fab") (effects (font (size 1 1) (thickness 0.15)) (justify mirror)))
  (pad "1" smd roundrect (at -0.825 0 90) (size 0.8 0.95) (layers "B.Cu" "B.Paste" "B.Mask") (roundrect_rratio 0.25) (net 42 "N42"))
  (pad "2" smd roundrect (at 0.825 0 90) (size 0.8 0.95) (layers "B.Cu" "B.Paste" "B.Mask") (roundrect_rratio 0.25) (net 53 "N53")))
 (gr_line (start 194.5 96.5) (end 194.5 140) (layer "Edge.Cuts") (width 0.1))
 (gr_line (start 104 140) (end 104 96.5) (layer "Edge.Cuts") (width 0.1))
 (gr_line (start 104 96.5) (end 194.5 96.5) (layer "Edge.Cuts") (width 0.1))
 (segment (start 131.15 108.675) (end 130.575 108.1) (width 0.25) (layer "B.Cu") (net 20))
 (segment (start 131.25 109.8) (end 131.15 109.7) (width 0.25) (layer "B.Cu") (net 20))
 (segment (start 133.375 109.8) (end 131.25 109.8) (width 0.25) (layer "B.Cu") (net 20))
 (segment (start 128.975 109.1) (end 129.575 109.1) (width 0.25) (layer "B.Cu") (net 20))
 (segment (start 128.35 109.725) (end 128.975 109.1) (width 0.25) (layer "B.Cu") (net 20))
 (segment (start 129.575 109.1) (end 130.575 108.1) (width 0.25) (layer "B.Cu") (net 20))
 (segment (start 131.15 109.7) (end 131.15 108.675) (width 0.25) (layer "B.Cu") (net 20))
 (segment (start 128.35 110.7) (end 128.35 109.725) (width 0.25) (layer "B.Cu") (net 20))
 (segment (start 110.95 117.7) (end 110.95 116.625) (width 0.25) (layer "B.Cu") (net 40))
 (segment (start 113.95 116.7) (end 113.75 116.5) (width 0.25) (layer "B.Cu") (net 40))
 (segment (start 110.95 116.625) (end 111.575 116) (width 0.25) (layer "B.Cu") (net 40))
 (segment (start 113.75 115.575) (end 113.175 115) (width 0.25) (layer "B.Cu") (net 40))
 (segment (start 112.175 116) (end 113.175 115) (width 0.25) (layer "B.Cu") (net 40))
 (segment (start 111.575 116) (end 112.175 116) (width 0.25) (layer "B.Cu") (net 40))
 (segment (start 113.75 116.5) (end 113.75 115.575) (width 0.25) (layer "B.Cu") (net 40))
 (segment (start 115.975 116.7) (end 113.95 116.7) (width 0.25) (layer "B.Cu") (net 40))
 (segment (start 108.525 130.65) (end 108.5 130.675) (width 0.25) (layer "B.Cu") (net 45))
 (segment (start 110.85 130.65) (end 108.525 130.65) (width 0.25) (layer "B.Cu") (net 45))
 (segment (start 110.85 129.875) (end 111.65 129.075) (width 0.25) (layer "B.Cu") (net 45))
 (segment (start 110.85 130.65) (end 110.85 129.875) (width 0.25) (layer "B.Cu") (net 45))
 (segment (start 110.1 127.525) (end 110.05 127.475) (width 0.25) (layer "B.Cu") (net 42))
 (segment (start 111.65 127.525) (end 110.1 127.525) (width 0.25) (layer "B.Cu") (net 42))
 (segment (start 134.95 109.775) (end 134.925 109.8) (width 0.25) (layer "B.Cu") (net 44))
 (segment (start 136.65 109.775) (end 136.65 108.3) (width 0.25) (layer "B.Cu") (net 44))
 (segment (start 134.975 111.4) (end 134.975 109.85) (width 0.25) (layer "B.Cu") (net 44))
 (segment (start 136.65 109.775) (end 134.95 109.775) (width 0.25) (layer "B.Cu") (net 44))
 (segment (start 134.975 109.85) (end 134.925 109.8) (width 0.25) (layer "B.Cu") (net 44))
 (segment (start 132.825 106.4) (end 132.825 107.4) (width 0.25) (layer "B.Cu") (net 39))
 (segment (start 132.825 107.4) (end 132.125 108.1) (width 0.25) (layer "B.Cu") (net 39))
 (segment (start 128.975 107.55) (end 130.125 106.4) (width 0.25) (layer "B.Cu") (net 39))
 (segment (start 130.125 106.4) (end 132.825 106.4) (width 0.25) (layer "B.Cu") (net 39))
 (segment (start 117.55 116.675) (end 117.525 116.7) (width 0.25) (layer "B.Cu") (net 48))
 (segment (start 119.25 116.675) (end 117.55 116.675) (width 0.25) (layer "B.Cu") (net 48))
 (segment (start 119.25 115.2) (end 119.25 116.675) (width 0.25) (layer "B.Cu") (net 48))
 (segment (start 117.575 116.75) (end 117.525 116.7) (width 0.25) (layer "B.Cu") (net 48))
 (segment (start 117.575 118.3) (end 117.575 116.75) (width 0.25) (layer "B.Cu") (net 48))
 (segment (start 115.425 114.3) (end 114.725 115) (width 0.25) (layer "B.Cu") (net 52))
 (segment (start 115.425 113.3) (end 112.675 113.3) (width 0.25) (layer "B.Cu") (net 52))
 (segment (start 112.675 113.3) (end 111.575 114.4) (width 0.25) (layer "B.Cu") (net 52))
 (segment (start 115.425 113.3) (end 115.425 114.3) (width 0.25) (layer "B.Cu") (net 52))
 (segment (start 111.5 134.175) (end 111.5 132.65) (width 0.25) (layer "B.Cu") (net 46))
 (segment (start 128.95 112.75) (end 129 112.7) (width 0.25) (layer "B.Cu") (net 50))
 (segment (start 128.95 114.375) (end 128.95 112.75) (width 0.25) (layer "B.Cu") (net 50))
 (segment (start 131.8 111.7) (end 133.025 111.7) (width 0.25) (layer "B.Cu") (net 43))
 (segment (start 133.025 111.7) (end 133.325 111.4) (width 0.25) (layer "B.Cu") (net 43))
 (segment (start 111.6 119.7) (end 111.6 121.325) (width 0.25) (layer "B.Cu") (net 53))
 (segment (start 111.6 121.325) (end 111.55 121.375) (width 0.25) (layer "B.Cu") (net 53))
 (segment (start 115.725 118.5) (end 115.925 118.3) (width 0.25) (layer "B.Cu") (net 49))
 (segment (start 114.4 118.5) (end 115.725 118.5) (width 0.25) (layer "B.Cu") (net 49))
 (segment (start 135.9 106.4) (end 136 106.3) (width 0.25) (layer "B.Cu") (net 51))
 (segment (start 134.475 106.4) (end 135.9 106.4) (width 0.25) (layer "B.Cu") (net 51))
 (segment (start 117.075 113.3) (end 118.5 113.3) (width 0.25) (layer "B.Cu") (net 47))
 (segment (start 118.5 113.3) (end 118.6 113.2) (width 0.25) (layer "B.Cu") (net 47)))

